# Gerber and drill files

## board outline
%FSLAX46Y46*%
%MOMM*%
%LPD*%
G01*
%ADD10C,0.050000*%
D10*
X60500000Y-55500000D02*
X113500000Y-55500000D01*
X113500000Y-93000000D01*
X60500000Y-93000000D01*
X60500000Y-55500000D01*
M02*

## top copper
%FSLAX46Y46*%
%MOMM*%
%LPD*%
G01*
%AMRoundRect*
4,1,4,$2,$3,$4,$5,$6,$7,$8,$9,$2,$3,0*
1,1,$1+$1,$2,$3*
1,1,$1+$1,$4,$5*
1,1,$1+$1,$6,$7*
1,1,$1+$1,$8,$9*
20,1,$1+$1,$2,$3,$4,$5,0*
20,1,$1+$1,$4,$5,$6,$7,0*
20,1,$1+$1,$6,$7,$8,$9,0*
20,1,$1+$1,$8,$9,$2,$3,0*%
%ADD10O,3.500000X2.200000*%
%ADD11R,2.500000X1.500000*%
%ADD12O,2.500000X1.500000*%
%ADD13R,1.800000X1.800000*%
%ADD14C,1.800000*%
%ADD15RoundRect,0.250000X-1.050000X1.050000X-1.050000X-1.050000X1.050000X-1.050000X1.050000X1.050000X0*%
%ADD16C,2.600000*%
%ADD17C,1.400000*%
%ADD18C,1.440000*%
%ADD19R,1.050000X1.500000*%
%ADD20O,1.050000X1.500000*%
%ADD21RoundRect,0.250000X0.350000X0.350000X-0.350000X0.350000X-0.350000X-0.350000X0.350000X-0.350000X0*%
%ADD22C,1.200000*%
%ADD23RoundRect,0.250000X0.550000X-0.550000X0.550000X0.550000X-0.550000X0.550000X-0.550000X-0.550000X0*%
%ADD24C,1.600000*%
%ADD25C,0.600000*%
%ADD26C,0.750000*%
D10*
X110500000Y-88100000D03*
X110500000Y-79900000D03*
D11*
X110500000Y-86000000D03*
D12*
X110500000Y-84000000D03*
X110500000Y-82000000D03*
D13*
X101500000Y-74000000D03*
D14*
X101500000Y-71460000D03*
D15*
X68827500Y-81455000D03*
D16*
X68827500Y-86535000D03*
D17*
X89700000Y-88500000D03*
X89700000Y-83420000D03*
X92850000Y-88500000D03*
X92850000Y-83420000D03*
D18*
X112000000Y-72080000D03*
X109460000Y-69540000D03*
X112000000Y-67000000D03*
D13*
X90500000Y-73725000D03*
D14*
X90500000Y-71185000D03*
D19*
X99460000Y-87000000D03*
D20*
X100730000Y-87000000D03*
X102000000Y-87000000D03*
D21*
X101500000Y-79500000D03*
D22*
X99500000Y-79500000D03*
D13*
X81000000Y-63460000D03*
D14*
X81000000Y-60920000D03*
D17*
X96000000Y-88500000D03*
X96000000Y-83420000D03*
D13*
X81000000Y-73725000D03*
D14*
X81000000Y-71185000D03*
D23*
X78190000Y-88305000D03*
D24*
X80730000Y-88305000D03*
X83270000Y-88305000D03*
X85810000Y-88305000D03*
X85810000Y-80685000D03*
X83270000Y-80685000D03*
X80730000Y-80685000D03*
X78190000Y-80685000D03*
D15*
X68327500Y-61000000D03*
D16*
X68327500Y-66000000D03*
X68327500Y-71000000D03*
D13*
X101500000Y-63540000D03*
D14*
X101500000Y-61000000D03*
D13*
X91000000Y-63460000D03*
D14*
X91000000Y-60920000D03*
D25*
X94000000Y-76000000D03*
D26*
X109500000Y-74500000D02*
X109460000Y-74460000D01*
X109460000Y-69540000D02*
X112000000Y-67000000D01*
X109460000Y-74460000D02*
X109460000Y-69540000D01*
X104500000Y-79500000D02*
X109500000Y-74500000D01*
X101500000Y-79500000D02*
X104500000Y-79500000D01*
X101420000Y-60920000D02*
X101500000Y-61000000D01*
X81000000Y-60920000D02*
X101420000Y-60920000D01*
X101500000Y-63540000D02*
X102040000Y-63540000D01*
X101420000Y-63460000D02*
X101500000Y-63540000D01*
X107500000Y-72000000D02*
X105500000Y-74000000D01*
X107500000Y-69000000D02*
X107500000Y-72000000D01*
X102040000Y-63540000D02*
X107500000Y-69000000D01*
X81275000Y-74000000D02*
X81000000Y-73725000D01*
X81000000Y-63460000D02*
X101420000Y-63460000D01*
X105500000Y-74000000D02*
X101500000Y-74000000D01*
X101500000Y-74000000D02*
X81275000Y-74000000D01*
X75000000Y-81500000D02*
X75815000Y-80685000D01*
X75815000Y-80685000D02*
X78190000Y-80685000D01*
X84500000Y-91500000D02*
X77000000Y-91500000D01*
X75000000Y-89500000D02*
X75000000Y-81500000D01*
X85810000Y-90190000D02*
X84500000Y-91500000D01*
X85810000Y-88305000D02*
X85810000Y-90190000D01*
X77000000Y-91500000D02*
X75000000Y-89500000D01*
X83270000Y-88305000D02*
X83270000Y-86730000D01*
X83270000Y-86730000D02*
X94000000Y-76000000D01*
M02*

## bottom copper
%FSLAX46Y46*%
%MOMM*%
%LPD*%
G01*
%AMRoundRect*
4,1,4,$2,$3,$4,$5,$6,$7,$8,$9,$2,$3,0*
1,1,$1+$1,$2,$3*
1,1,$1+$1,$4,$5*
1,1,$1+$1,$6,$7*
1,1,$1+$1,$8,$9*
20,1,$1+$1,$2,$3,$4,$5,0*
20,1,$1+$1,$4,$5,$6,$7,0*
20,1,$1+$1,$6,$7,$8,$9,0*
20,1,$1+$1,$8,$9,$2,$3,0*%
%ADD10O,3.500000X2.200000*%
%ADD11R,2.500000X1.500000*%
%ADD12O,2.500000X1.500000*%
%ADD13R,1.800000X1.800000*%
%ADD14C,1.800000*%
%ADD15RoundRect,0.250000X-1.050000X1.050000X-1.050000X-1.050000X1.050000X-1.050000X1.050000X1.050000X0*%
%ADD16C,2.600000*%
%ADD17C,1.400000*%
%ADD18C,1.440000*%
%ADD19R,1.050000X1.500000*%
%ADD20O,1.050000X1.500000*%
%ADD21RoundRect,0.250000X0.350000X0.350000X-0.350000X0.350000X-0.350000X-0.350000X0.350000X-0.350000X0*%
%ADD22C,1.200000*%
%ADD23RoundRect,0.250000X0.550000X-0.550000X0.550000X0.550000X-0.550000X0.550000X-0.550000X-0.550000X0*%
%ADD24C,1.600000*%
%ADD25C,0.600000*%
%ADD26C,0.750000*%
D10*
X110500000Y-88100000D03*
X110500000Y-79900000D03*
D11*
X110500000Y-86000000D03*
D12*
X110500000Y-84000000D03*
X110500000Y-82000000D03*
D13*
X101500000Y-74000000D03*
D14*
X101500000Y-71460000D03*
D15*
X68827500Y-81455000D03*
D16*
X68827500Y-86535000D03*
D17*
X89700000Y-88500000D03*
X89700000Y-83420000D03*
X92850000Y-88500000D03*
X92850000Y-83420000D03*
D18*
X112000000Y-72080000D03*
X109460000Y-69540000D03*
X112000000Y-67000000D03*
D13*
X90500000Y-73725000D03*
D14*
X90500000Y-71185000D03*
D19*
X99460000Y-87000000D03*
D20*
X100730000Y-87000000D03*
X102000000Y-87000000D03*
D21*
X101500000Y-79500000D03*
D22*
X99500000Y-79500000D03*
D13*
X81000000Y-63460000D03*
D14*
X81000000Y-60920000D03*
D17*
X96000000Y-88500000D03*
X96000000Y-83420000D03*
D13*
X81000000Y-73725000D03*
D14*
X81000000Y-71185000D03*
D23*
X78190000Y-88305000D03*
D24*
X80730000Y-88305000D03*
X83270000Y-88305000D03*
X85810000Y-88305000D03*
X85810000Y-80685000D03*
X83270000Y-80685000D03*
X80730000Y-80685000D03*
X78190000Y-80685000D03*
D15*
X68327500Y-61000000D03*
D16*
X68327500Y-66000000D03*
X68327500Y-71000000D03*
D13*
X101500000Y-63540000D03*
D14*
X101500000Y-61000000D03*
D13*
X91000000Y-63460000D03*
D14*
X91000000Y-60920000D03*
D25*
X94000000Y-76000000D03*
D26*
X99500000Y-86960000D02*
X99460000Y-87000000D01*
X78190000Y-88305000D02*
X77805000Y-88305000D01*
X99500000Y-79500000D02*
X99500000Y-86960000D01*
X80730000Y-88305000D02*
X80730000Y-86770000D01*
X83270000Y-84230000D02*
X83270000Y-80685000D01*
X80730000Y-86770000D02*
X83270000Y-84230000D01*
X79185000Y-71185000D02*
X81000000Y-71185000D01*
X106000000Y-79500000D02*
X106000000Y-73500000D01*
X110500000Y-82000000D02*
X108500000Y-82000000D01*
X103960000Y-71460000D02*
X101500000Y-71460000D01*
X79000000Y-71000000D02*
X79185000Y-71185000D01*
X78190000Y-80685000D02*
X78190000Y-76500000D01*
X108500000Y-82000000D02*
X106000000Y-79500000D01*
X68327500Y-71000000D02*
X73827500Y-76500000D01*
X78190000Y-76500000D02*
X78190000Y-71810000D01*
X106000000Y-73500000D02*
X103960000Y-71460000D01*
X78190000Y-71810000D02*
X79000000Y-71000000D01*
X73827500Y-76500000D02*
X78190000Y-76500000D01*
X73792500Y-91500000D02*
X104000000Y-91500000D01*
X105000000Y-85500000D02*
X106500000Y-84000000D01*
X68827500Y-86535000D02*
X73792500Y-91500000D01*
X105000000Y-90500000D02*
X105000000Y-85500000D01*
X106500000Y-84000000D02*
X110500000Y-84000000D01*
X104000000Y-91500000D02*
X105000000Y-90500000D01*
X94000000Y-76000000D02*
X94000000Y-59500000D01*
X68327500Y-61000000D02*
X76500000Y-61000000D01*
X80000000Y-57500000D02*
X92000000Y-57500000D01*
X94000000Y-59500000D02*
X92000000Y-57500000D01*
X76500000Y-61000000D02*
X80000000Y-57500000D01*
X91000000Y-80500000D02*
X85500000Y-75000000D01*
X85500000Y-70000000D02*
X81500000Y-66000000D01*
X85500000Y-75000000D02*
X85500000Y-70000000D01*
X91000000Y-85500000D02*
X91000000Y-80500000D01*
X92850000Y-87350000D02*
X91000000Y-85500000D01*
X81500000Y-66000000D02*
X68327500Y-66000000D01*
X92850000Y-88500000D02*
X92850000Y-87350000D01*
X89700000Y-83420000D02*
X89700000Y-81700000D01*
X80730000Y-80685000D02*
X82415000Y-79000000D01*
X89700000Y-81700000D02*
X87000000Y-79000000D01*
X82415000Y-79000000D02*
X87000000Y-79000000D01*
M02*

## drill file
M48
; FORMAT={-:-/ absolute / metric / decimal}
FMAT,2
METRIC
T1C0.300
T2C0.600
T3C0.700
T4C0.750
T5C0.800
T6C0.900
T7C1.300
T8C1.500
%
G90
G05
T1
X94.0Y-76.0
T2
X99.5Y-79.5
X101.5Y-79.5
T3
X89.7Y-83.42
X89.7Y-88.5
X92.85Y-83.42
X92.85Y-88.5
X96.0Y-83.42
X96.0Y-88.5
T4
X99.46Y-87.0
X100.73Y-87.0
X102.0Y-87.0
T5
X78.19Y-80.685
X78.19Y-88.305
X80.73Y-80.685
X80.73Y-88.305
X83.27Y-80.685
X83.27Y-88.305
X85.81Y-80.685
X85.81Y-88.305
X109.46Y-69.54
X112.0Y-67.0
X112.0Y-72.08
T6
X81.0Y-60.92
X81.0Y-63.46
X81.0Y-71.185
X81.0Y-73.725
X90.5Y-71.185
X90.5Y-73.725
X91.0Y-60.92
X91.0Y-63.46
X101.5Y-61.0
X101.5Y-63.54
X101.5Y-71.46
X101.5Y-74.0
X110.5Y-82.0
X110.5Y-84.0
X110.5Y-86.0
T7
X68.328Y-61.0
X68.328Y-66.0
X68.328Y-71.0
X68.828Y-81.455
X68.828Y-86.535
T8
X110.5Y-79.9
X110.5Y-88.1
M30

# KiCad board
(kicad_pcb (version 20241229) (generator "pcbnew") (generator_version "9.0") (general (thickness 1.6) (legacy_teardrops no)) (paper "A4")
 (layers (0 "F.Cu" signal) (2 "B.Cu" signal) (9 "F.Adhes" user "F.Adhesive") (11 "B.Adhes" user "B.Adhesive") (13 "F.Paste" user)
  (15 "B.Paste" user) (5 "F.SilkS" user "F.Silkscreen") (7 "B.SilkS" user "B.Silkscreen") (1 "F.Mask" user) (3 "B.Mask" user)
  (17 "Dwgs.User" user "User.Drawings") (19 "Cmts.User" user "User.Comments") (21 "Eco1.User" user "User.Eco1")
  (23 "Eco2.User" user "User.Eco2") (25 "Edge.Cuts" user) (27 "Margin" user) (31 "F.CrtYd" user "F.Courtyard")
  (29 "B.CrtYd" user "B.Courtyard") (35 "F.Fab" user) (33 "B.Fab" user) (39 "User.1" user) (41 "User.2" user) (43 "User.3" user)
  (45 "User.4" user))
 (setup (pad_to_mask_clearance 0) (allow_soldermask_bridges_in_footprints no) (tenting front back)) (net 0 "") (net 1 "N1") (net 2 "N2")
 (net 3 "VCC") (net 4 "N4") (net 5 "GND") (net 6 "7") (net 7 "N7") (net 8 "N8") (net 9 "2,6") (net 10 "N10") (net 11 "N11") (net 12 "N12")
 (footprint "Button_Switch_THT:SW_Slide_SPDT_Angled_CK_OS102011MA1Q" (layer "F.Cu") (at 110.5 86 90)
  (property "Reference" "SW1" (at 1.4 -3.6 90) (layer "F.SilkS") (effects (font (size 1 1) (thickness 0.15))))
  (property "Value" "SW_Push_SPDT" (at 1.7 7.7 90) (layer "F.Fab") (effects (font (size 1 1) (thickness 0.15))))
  (pad "" thru_hole oval (at -2.1 0 90) (size 2.2 3.5) (drill 1.5) (layers "*.Cu" "*.Mask") (remove_unused_layers no))
  (pad "" thru_hole oval (at 6.1 0 90) (size 2.2 3.5) (drill 1.5) (layers "*.Cu" "*.Mask") (remove_unused_layers no))
  (pad "1" thru_hole rect (at 0 0 90) (size 1.5 2.5) (drill 0.9) (layers "*.Cu" "*.Mask") (remove_unused_layers no) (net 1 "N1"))
  (pad "2" thru_hole oval (at 2 0 90) (size 1.5 2.5) (drill 0.9) (layers "*.Cu" "*.Mask") (remove_unused_layers no) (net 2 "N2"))
  (pad "3" thru_hole oval (at 4 0 90) (size 1.5 2.5) (drill 0.9) (layers "*.Cu" "*.Mask") (remove_unused_layers no) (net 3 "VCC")))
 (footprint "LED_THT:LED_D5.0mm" (layer "F.Cu") (at 101.5 74 90)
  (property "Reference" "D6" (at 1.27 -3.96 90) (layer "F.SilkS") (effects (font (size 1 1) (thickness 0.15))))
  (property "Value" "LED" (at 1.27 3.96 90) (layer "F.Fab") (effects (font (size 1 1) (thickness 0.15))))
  (pad "1" thru_hole rect (at 0 0 90) (size 1.8 1.8) (drill 0.9) (layers "*.Cu" "*.Mask") (remove_unused_layers no) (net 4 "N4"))
  (pad "2" thru_hole circle (at 2.54 0 90) (size 1.8 1.8) (drill 0.9) (layers "*.Cu" "*.Mask") (remove_unused_layers no) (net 3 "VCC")))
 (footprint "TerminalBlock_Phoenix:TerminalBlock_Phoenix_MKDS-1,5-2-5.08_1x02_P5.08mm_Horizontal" (layer "F.Cu") (at 68.8275 81.455 -90)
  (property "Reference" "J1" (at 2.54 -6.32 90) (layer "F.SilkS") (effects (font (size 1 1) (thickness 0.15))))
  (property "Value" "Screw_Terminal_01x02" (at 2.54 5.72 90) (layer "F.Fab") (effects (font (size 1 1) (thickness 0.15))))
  (pad "1" thru_hole roundrect (at 0 0 270) (size 2.6 2.6) (drill 1.3) (layers "*.Cu" "*.Mask") (remove_unused_layers no)
   (roundrect_rratio 0.096154) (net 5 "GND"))
  (pad "2" thru_hole circle (at 5.08 0 270) (size 2.6 2.6) (drill 1.3) (layers "*.Cu" "*.Mask") (remove_unused_layers no) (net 2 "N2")))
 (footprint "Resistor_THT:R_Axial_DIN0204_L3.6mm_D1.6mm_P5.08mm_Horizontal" (layer "F.Cu") (at 89.7 88.5 90)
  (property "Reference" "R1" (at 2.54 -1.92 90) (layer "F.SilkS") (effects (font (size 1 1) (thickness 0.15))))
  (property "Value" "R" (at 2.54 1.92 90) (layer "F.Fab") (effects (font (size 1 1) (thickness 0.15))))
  (pad "1" thru_hole circle (at 0 0 90) (size 1.4 1.4) (drill 0.7) (layers "*.Cu" "*.Mask") (remove_unused_layers no) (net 3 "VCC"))
  (pad "2" thru_hole circle (at 5.08 0 90) (size 1.4 1.4) (drill 0.7) (layers "*.Cu" "*.Mask") (remove_unused_layers no) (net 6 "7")))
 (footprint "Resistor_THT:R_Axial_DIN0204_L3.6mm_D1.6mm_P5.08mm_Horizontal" (layer "F.Cu") (at 92.85 88.5 90)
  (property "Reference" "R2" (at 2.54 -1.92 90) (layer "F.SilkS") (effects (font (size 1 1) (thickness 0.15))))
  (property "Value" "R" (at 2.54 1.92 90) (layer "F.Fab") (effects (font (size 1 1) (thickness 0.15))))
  (pad "1" thru_hole circle (at 0 0 90) (size 1.4 1.4) (drill 0.7) (layers "*.Cu" "*.Mask") (remove_unused_layers no) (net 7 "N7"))
  (pad "2" thru_hole circle (at 5.08 0 90) (size 1.4 1.4) (drill 0.7) (layers "*.Cu" "*.Mask") (remove_unused_layers no) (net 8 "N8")))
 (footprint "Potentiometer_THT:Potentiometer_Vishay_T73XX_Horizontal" (layer "F.Cu") (at 112 72.08 180)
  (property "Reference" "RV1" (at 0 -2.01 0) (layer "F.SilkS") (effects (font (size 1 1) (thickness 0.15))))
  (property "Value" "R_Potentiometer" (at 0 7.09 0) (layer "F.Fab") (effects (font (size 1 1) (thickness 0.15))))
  (pad "1" thru_hole circle (at 0 0 180) (size 1.44 1.44) (drill 0.8) (layers "*.Cu" "*.Mask") (remove_unused_layers no) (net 6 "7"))
  (pad "2" thru_hole circle (at 2.54 2.54 180) (size 1.44 1.44) (drill 0.8) (layers "*.Cu" "*.Mask") (remove_unused_layers no) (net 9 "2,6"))
  (pad "3" thru_hole circle (at 0 5.08 180) (size 1.44 1.44) (drill 0.8) (layers "*.Cu" "*.Mask") (remove_unused_layers no) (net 9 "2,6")))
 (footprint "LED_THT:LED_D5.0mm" (layer "F.Cu") (at 90.5 73.725 90)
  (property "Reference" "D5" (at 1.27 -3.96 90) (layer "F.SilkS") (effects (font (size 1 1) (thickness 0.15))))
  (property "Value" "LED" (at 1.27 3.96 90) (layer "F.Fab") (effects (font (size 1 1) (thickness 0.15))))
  (pad "1" thru_hole rect (at 0 0 90) (size 1.8 1.8) (drill 0.9) (layers "*.Cu" "*.Mask") (remove_unused_layers no) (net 4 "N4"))
  (pad "2" thru_hole circle (at 2.54 0 90) (size 1.8 1.8) (drill 0.9) (layers "*.Cu" "*.Mask") (remove_unused_layers no) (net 3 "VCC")))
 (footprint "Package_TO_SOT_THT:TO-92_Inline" (layer "F.Cu") (at 99.46 87)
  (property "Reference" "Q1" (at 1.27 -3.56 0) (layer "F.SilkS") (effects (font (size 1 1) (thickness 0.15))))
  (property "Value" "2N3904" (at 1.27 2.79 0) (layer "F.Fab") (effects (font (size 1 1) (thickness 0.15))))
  (pad "1" thru_hole rect (at 0 0) (size 1.05 1.5) (drill 0.75) (layers "*.Cu" "*.Mask") (remove_unused_layers no) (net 5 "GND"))
  (pad "2" thru_hole oval (at 1.27 0) (size 1.05 1.5) (drill 0.75) (layers "*.Cu" "*.Mask") (remove_unused_layers no) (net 8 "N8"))
  (pad "3" thru_hole oval (at 2.54 0) (size 1.05 1.5) (drill 0.75) (layers "*.Cu" "*.Mask") (remove_unused_layers no) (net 4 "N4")))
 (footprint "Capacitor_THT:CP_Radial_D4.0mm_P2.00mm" (layer "F.Cu") (at 101.5 79.5 180)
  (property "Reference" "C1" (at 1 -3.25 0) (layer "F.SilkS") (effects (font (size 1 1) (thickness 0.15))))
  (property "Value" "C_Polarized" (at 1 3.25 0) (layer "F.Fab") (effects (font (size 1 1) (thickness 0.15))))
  (pad "1" thru_hole roundrect (at 0 0 180) (size 1.2 1.2) (drill 0.6) (layers "*.Cu" "*.Mask") (remove_unused_layers no)
   (roundrect_rratio 0.208333) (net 9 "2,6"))
  (pad "2" thru_hole circle (at 2 0 180) (size 1.2 1.2) (drill 0.6) (layers "*.Cu" "*.Mask") (remove_unused_layers no) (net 5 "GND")))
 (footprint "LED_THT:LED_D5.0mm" (layer "F.Cu") (at 81 63.46 90)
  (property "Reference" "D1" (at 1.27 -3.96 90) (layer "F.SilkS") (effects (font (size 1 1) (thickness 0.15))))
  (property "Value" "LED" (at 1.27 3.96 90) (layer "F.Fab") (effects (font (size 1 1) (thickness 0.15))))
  (pad "1" thru_hole rect (at 0 0 90) (size 1.8 1.8) (drill 0.9) (layers "*.Cu" "*.Mask") (remove_unused_layers no) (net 4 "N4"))
  (pad "2" thru_hole circle (at 2.54 0 90) (size 1.8 1.8) (drill 0.9) (layers "*.Cu" "*.Mask") (remove_unused_layers no) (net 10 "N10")))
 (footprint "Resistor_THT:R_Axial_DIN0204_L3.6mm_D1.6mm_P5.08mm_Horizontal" (layer "F.Cu") (at 96 88.5 90)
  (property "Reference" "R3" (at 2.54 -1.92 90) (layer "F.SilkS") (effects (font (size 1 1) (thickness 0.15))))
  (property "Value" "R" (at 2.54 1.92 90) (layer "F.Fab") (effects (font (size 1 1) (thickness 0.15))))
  (pad "1" thru_hole circle (at 0 0 90) (size 1.4 1.4) (drill 0.7) (layers "*.Cu" "*.Mask") (remove_unused_layers no) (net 3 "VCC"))
  (pad "2" thru_hole circle (at 5.08 0 90) (size 1.4 1.4) (drill 0.7) (layers "*.Cu" "*.Mask") (remove_unused_layers no) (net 10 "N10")))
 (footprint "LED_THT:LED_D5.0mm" (layer "F.Cu") (at 81 73.725 90)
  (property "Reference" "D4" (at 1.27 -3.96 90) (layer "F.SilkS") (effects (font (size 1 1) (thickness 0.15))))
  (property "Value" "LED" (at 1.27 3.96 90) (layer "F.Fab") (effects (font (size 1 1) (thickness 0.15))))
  (pad "1" thru_hole rect (at 0 0 90) (size 1.8 1.8) (drill 0.9) (layers "*.Cu" "*.Mask") (remove_unused_layers no) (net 4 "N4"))
  (pad "2" thru_hole circle (at 2.54 0 90) (size 1.8 1.8) (drill 0.9) (layers "*.Cu" "*.Mask") (remove_unused_layers no) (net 3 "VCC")))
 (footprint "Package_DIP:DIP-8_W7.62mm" (layer "F.Cu") (at 78.19 88.305 90)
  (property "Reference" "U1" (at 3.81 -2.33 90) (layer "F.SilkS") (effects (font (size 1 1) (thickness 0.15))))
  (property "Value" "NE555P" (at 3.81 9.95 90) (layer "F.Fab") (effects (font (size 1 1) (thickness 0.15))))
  (pad "1" thru_hole roundrect (at 0 0 90) (size 1.6 1.6) (drill 0.8) (layers "*.Cu" "*.Mask") (remove_unused_layers no)
   (roundrect_rratio 0.15625) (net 5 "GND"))
  (pad "2" thru_hole circle (at 0 2.54 90) (size 1.6 1.6) (drill 0.8) (layers "*.Cu" "*.Mask") (remove_unused_layers no) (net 9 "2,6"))
  (pad "3" thru_hole circle (at 0 5.08 90) (size 1.6 1.6) (drill 0.8) (layers "*.Cu" "*.Mask") (remove_unused_layers no) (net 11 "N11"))
  (pad "4" thru_hole circle (at 0 7.62 90) (size 1.6 1.6) (drill 0.8) (layers "*.Cu" "*.Mask") (remove_unused_layers no) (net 3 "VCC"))
  (pad "5" thru_hole circle (at 7.62 7.62 90) (size 1.6 1.6) (drill 0.8) (layers "*.Cu" "*.Mask") (remove_unused_layers no) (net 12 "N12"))
  (pad "6" thru_hole circle (at 7.62 5.08 90) (size 1.6 1.6) (drill 0.8) (layers "*.Cu" "*.Mask") (remove_unused_layers no) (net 9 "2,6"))
  (pad "7" thru_hole circle (at 7.62 2.54 90) (size 1.6 1.6) (drill 0.8) (layers "*.Cu" "*.Mask") (remove_unused_layers no) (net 6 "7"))
  (pad "8" thru_hole circle (at 7.62 0 90) (size 1.6 1.6) (drill 0.8) (layers "*.Cu" "*.Mask") (remove_unused_layers no) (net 3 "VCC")))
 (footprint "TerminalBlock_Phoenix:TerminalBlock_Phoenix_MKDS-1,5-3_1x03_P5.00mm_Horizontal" (layer "F.Cu") (at 68.3275 61 -90)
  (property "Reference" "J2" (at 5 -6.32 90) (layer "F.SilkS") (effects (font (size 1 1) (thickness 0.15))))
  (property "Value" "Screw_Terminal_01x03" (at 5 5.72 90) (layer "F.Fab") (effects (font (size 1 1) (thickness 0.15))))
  (pad "1" thru_hole roundrect (at 0 0 270) (size 2.6 2.6) (drill 1.3) (layers "*.Cu" "*.Mask") (remove_unused_layers no)
   (roundrect_rratio 0.096154) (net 11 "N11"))
  (pad "2" thru_hole circle (at 5 0 270) (size 2.6 2.6) (drill 1.3) (layers "*.Cu" "*.Mask") (remove_unused_layers no) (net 7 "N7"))
  (pad "3" thru_hole circle (at 10 0 270) (size 2.6 2.6) (drill 1.3) (layers "*.Cu" "*.Mask") (remove_unused_layers no) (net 3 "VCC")))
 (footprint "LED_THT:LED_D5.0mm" (layer "F.Cu") (at 101.5 63.54 90)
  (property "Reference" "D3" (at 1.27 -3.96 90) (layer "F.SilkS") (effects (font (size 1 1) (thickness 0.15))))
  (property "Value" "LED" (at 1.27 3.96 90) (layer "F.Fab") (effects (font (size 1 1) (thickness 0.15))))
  (pad "1" thru_hole rect (at 0 0 90) (size 1.8 1.8) (drill 0.9) (layers "*.Cu" "*.Mask") (remove_unused_layers no) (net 4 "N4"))
  (pad "2" thru_hole circle (at 2.54 0 90) (size 1.8 1.8) (drill 0.9) (layers "*.Cu" "*.Mask") (remove_unused_layers no) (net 10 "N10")))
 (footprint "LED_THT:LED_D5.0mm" (layer "F.Cu") (at 91 63.46 90)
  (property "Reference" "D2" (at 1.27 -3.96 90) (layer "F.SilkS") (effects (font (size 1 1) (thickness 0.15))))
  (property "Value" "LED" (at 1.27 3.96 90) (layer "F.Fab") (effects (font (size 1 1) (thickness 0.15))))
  (pad "1" thru_hole rect (at 0 0 90) (size 1.8 1.8) (drill 0.9) (layers "*.Cu" "*.Mask") (remove_unused_layers no) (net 4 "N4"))
  (pad "2" thru_hole circle (at 2.54 0 90) (size 1.8 1.8) (drill 0.9) (layers "*.Cu" "*.Mask") (remove_unused_layers no) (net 10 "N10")))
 (gr_rect (start 60.5 55.5) (end 113.5 93) (stroke (width 0.05) (type default)) (fill no) (layer "Edge.Cuts"))
 (segment (start 99.5 86.96) (end 99.46 87) (width 0.75) (layer "B.Cu") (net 5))
 (segment (start 78.19 88.305) (end 77.805 88.305) (width 0.75) (layer "B.Cu") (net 5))
 (segment (start 99.5 79.5) (end 99.5 86.96) (width 0.75) (layer "B.Cu") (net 5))
 (segment (start 109.5 74.5) (end 109.46 74.46) (width 0.75) (layer "F.Cu") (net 9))
 (segment (start 109.46 69.54) (end 112 67) (width 0.75) (layer "F.Cu") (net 9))
 (segment (start 109.46 74.46) (end 109.46 69.54) (width 0.75) (layer "F.Cu") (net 9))
 (segment (start 104.5 79.5) (end 109.5 74.5) (width 0.75) (layer "F.Cu") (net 9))
 (segment (start 101.5 79.5) (end 104.5 79.5) (width 0.75) (layer "F.Cu") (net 9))
 (segment (start 80.73 88.305) (end 80.73 86.77) (width 0.75) (layer "B.Cu") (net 9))
 (segment (start 83.27 84.23) (end 83.27 80.685) (width 0.75) (layer "B.Cu") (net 9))
 (segment (start 80.73 86.77) (end 83.27 84.23) (width 0.75) (layer "B.Cu") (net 9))
 (segment (start 101.42 60.92) (end 101.5 61) (width 0.75) (layer "F.Cu") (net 10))
 (segment (start 81 60.92) (end 101.42 60.92) (width 0.75) (layer "F.Cu") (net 10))
 (segment (start 101.5 63.54) (end 102.04 63.54) (width 0.75) (layer "F.Cu") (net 4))
 (segment (start 101.42 63.46) (end 101.5 63.54) (width 0.75) (layer "F.Cu") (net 4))
 (segment (start 107.5 72) (end 105.5 74) (width 0.75) (layer "F.Cu") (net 4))
 (segment (start 107.5 69) (end 107.5 72) (width 0.75) (layer "F.Cu") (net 4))
 (segment (start 102.04 63.54) (end 107.5 69) (width 0.75) (layer "F.Cu") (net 4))
 (segment (start 81.275 74) (end 81 73.725) (width 0.75) (layer "F.Cu") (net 4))
 (segment (start 81 63.46) (end 101.42 63.46) (width 0.75) (layer "F.Cu") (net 4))
 (segment (start 105.5 74) (end 101.5 74) (width 0.75) (layer "F.Cu") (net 4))
 (segment (start 101.5 74) (end 81.275 74) (width 0.75) (layer "F.Cu") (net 4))
 (segment (start 75 81.5) (end 75.815 80.685) (width 0.75) (layer "F.Cu") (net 3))
 (segment (start 75.815 80.685) (end 78.19 80.685) (width 0.75) (layer "F.Cu") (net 3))
 (segment (start 84.5 91.5) (end 77 91.5) (width 0.75) (layer "F.Cu") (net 3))
 (segment (start 75 89.5) (end 75 81.5) (width 0.75) (layer "F.Cu") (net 3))
 (segment (start 85.81 90.19) (end 84.5 91.5) (width 0.75) (layer "F.Cu") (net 3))
 (segment (start 85.81 88.305) (end 85.81 90.19) (width 0.75) (layer "F.Cu") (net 3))
 (segment (start 77 91.5) (end 75 89.5) (width 0.75) (layer "F.Cu") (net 3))
 (segment (start 79.185 71.185) (end 81 71.185) (width 0.75) (layer "B.Cu") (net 3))
 (segment (start 106 79.5) (end 106 73.5) (width 0.75) (layer "B.Cu") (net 3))
 (segment (start 110.5 82) (end 108.5 82) (width 0.75) (layer "B.Cu") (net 3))
 (segment (start 103.96 71.46) (end 101.5 71.46) (width 0.75) (layer "B.Cu") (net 3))
 (segment (start 79 71) (end 79.185 71.185) (width 0.75) (layer "B.Cu") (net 3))
 (segment (start 78.19 80.685) (end 78.19 76.5) (width 0.75) (layer "B.Cu") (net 3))
 (segment (start 108.5 82) (end 106 79.5) (width 0.75) (layer "B.Cu") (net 3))
 (segment (start 68.3275 71) (end 73.8275 76.5) (width 0.75) (layer "B.Cu") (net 3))
 (segment (start 78.19 76.5) (end 78.19 71.81) (width 0.75) (layer "B.Cu") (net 3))
 (segment (start 106 73.5) (end 103.96 71.46) (width 0.75) (layer "B.Cu") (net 3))
 (segment (start 78.19 71.81) (end 79 71) (width 0.75) (layer "B.Cu") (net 3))
 (segment (start 73.8275 76.5) (end 78.19 76.5) (width 0.75) (layer "B.Cu") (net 3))
 (segment (start 73.7925 91.5) (end 104 91.5) (width 0.75) (layer "B.Cu") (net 2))
 (segment (start 105 85.5) (end 106.5 84) (width 0.75) (layer "B.Cu") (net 2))
 (segment (start 68.8275 86.535) (end 73.7925 91.5) (width 0.75) (layer "B.Cu") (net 2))
 (segment (start 105 90.5) (end 105 85.5) (width 0.75) (layer "B.Cu") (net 2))
 (segment (start 106.5 84) (end 110.5 84) (width 0.75) (layer "B.Cu") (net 2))
 (segment (start 104 91.5) (end 105 90.5) (width 0.75) (layer "B.Cu") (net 2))
 (segment (start 83.27 88.305) (end 83.27 86.73) (width 0.75) (layer "F.Cu") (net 11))
 (segment (start 83.27 86.73) (end 94 76) (width 0.75) (layer "F.Cu") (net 11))
 (via (at 94 76) (size 0.6) (drill 0.3) (layers "F.Cu" "B.Cu") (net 11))
 (segment (start 94 76) (end 94 59.5) (width 0.75) (layer "B.Cu") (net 11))
 (segment (start 68.3275 61) (end 76.5 61) (width 0.75) (layer "B.Cu") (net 11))
 (segment (start 80 57.5) (end 92 57.5) (width 0.75) (layer "B.Cu") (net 11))
 (segment (start 94 59.5) (end 92 57.5) (width 0.75) (layer "B.Cu") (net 11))
 (segment (start 76.5 61) (end 80 57.5) (width 0.75) (layer "B.Cu") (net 11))
 (segment (start 91 80.5) (end 85.5 75) (width 0.75) (layer "B.Cu") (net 7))
 (segment (start 85.5 70) (end 81.5 66) (width 0.75) (layer "B.Cu") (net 7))
 (segment (start 85.5 75) (end 85.5 70) (width 0.75) (layer "B.Cu") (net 7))
 (segment (start 91 85.5) (end 91 80.5) (width 0.75) (layer "B.Cu") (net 7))
 (segment (start 92.85 87.35) (end 91 85.5) (width 0.75) (layer "B.Cu") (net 7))
 (segment (start 81.5 66) (end 68.3275 66) (width 0.75) (layer "B.Cu") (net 7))
 (segment (start 92.85 88.5) (end 92.85 87.35) (width 0.75) (layer "B.Cu") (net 7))
 (segment (start 89.7 83.42) (end 89.7 81.7) (width 0.75) (layer "B.Cu") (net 6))
 (segment (start 80.73 80.685) (end 82.415 79) (width 0.75) (layer "B.Cu") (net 6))
 (segment (start 89.7 81.7) (end 87 79) (width 0.75) (layer "B.Cu") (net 6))
 (segment (start 82.415 79) (end 87 79) (width 0.75) (layer "B.Cu") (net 6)))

